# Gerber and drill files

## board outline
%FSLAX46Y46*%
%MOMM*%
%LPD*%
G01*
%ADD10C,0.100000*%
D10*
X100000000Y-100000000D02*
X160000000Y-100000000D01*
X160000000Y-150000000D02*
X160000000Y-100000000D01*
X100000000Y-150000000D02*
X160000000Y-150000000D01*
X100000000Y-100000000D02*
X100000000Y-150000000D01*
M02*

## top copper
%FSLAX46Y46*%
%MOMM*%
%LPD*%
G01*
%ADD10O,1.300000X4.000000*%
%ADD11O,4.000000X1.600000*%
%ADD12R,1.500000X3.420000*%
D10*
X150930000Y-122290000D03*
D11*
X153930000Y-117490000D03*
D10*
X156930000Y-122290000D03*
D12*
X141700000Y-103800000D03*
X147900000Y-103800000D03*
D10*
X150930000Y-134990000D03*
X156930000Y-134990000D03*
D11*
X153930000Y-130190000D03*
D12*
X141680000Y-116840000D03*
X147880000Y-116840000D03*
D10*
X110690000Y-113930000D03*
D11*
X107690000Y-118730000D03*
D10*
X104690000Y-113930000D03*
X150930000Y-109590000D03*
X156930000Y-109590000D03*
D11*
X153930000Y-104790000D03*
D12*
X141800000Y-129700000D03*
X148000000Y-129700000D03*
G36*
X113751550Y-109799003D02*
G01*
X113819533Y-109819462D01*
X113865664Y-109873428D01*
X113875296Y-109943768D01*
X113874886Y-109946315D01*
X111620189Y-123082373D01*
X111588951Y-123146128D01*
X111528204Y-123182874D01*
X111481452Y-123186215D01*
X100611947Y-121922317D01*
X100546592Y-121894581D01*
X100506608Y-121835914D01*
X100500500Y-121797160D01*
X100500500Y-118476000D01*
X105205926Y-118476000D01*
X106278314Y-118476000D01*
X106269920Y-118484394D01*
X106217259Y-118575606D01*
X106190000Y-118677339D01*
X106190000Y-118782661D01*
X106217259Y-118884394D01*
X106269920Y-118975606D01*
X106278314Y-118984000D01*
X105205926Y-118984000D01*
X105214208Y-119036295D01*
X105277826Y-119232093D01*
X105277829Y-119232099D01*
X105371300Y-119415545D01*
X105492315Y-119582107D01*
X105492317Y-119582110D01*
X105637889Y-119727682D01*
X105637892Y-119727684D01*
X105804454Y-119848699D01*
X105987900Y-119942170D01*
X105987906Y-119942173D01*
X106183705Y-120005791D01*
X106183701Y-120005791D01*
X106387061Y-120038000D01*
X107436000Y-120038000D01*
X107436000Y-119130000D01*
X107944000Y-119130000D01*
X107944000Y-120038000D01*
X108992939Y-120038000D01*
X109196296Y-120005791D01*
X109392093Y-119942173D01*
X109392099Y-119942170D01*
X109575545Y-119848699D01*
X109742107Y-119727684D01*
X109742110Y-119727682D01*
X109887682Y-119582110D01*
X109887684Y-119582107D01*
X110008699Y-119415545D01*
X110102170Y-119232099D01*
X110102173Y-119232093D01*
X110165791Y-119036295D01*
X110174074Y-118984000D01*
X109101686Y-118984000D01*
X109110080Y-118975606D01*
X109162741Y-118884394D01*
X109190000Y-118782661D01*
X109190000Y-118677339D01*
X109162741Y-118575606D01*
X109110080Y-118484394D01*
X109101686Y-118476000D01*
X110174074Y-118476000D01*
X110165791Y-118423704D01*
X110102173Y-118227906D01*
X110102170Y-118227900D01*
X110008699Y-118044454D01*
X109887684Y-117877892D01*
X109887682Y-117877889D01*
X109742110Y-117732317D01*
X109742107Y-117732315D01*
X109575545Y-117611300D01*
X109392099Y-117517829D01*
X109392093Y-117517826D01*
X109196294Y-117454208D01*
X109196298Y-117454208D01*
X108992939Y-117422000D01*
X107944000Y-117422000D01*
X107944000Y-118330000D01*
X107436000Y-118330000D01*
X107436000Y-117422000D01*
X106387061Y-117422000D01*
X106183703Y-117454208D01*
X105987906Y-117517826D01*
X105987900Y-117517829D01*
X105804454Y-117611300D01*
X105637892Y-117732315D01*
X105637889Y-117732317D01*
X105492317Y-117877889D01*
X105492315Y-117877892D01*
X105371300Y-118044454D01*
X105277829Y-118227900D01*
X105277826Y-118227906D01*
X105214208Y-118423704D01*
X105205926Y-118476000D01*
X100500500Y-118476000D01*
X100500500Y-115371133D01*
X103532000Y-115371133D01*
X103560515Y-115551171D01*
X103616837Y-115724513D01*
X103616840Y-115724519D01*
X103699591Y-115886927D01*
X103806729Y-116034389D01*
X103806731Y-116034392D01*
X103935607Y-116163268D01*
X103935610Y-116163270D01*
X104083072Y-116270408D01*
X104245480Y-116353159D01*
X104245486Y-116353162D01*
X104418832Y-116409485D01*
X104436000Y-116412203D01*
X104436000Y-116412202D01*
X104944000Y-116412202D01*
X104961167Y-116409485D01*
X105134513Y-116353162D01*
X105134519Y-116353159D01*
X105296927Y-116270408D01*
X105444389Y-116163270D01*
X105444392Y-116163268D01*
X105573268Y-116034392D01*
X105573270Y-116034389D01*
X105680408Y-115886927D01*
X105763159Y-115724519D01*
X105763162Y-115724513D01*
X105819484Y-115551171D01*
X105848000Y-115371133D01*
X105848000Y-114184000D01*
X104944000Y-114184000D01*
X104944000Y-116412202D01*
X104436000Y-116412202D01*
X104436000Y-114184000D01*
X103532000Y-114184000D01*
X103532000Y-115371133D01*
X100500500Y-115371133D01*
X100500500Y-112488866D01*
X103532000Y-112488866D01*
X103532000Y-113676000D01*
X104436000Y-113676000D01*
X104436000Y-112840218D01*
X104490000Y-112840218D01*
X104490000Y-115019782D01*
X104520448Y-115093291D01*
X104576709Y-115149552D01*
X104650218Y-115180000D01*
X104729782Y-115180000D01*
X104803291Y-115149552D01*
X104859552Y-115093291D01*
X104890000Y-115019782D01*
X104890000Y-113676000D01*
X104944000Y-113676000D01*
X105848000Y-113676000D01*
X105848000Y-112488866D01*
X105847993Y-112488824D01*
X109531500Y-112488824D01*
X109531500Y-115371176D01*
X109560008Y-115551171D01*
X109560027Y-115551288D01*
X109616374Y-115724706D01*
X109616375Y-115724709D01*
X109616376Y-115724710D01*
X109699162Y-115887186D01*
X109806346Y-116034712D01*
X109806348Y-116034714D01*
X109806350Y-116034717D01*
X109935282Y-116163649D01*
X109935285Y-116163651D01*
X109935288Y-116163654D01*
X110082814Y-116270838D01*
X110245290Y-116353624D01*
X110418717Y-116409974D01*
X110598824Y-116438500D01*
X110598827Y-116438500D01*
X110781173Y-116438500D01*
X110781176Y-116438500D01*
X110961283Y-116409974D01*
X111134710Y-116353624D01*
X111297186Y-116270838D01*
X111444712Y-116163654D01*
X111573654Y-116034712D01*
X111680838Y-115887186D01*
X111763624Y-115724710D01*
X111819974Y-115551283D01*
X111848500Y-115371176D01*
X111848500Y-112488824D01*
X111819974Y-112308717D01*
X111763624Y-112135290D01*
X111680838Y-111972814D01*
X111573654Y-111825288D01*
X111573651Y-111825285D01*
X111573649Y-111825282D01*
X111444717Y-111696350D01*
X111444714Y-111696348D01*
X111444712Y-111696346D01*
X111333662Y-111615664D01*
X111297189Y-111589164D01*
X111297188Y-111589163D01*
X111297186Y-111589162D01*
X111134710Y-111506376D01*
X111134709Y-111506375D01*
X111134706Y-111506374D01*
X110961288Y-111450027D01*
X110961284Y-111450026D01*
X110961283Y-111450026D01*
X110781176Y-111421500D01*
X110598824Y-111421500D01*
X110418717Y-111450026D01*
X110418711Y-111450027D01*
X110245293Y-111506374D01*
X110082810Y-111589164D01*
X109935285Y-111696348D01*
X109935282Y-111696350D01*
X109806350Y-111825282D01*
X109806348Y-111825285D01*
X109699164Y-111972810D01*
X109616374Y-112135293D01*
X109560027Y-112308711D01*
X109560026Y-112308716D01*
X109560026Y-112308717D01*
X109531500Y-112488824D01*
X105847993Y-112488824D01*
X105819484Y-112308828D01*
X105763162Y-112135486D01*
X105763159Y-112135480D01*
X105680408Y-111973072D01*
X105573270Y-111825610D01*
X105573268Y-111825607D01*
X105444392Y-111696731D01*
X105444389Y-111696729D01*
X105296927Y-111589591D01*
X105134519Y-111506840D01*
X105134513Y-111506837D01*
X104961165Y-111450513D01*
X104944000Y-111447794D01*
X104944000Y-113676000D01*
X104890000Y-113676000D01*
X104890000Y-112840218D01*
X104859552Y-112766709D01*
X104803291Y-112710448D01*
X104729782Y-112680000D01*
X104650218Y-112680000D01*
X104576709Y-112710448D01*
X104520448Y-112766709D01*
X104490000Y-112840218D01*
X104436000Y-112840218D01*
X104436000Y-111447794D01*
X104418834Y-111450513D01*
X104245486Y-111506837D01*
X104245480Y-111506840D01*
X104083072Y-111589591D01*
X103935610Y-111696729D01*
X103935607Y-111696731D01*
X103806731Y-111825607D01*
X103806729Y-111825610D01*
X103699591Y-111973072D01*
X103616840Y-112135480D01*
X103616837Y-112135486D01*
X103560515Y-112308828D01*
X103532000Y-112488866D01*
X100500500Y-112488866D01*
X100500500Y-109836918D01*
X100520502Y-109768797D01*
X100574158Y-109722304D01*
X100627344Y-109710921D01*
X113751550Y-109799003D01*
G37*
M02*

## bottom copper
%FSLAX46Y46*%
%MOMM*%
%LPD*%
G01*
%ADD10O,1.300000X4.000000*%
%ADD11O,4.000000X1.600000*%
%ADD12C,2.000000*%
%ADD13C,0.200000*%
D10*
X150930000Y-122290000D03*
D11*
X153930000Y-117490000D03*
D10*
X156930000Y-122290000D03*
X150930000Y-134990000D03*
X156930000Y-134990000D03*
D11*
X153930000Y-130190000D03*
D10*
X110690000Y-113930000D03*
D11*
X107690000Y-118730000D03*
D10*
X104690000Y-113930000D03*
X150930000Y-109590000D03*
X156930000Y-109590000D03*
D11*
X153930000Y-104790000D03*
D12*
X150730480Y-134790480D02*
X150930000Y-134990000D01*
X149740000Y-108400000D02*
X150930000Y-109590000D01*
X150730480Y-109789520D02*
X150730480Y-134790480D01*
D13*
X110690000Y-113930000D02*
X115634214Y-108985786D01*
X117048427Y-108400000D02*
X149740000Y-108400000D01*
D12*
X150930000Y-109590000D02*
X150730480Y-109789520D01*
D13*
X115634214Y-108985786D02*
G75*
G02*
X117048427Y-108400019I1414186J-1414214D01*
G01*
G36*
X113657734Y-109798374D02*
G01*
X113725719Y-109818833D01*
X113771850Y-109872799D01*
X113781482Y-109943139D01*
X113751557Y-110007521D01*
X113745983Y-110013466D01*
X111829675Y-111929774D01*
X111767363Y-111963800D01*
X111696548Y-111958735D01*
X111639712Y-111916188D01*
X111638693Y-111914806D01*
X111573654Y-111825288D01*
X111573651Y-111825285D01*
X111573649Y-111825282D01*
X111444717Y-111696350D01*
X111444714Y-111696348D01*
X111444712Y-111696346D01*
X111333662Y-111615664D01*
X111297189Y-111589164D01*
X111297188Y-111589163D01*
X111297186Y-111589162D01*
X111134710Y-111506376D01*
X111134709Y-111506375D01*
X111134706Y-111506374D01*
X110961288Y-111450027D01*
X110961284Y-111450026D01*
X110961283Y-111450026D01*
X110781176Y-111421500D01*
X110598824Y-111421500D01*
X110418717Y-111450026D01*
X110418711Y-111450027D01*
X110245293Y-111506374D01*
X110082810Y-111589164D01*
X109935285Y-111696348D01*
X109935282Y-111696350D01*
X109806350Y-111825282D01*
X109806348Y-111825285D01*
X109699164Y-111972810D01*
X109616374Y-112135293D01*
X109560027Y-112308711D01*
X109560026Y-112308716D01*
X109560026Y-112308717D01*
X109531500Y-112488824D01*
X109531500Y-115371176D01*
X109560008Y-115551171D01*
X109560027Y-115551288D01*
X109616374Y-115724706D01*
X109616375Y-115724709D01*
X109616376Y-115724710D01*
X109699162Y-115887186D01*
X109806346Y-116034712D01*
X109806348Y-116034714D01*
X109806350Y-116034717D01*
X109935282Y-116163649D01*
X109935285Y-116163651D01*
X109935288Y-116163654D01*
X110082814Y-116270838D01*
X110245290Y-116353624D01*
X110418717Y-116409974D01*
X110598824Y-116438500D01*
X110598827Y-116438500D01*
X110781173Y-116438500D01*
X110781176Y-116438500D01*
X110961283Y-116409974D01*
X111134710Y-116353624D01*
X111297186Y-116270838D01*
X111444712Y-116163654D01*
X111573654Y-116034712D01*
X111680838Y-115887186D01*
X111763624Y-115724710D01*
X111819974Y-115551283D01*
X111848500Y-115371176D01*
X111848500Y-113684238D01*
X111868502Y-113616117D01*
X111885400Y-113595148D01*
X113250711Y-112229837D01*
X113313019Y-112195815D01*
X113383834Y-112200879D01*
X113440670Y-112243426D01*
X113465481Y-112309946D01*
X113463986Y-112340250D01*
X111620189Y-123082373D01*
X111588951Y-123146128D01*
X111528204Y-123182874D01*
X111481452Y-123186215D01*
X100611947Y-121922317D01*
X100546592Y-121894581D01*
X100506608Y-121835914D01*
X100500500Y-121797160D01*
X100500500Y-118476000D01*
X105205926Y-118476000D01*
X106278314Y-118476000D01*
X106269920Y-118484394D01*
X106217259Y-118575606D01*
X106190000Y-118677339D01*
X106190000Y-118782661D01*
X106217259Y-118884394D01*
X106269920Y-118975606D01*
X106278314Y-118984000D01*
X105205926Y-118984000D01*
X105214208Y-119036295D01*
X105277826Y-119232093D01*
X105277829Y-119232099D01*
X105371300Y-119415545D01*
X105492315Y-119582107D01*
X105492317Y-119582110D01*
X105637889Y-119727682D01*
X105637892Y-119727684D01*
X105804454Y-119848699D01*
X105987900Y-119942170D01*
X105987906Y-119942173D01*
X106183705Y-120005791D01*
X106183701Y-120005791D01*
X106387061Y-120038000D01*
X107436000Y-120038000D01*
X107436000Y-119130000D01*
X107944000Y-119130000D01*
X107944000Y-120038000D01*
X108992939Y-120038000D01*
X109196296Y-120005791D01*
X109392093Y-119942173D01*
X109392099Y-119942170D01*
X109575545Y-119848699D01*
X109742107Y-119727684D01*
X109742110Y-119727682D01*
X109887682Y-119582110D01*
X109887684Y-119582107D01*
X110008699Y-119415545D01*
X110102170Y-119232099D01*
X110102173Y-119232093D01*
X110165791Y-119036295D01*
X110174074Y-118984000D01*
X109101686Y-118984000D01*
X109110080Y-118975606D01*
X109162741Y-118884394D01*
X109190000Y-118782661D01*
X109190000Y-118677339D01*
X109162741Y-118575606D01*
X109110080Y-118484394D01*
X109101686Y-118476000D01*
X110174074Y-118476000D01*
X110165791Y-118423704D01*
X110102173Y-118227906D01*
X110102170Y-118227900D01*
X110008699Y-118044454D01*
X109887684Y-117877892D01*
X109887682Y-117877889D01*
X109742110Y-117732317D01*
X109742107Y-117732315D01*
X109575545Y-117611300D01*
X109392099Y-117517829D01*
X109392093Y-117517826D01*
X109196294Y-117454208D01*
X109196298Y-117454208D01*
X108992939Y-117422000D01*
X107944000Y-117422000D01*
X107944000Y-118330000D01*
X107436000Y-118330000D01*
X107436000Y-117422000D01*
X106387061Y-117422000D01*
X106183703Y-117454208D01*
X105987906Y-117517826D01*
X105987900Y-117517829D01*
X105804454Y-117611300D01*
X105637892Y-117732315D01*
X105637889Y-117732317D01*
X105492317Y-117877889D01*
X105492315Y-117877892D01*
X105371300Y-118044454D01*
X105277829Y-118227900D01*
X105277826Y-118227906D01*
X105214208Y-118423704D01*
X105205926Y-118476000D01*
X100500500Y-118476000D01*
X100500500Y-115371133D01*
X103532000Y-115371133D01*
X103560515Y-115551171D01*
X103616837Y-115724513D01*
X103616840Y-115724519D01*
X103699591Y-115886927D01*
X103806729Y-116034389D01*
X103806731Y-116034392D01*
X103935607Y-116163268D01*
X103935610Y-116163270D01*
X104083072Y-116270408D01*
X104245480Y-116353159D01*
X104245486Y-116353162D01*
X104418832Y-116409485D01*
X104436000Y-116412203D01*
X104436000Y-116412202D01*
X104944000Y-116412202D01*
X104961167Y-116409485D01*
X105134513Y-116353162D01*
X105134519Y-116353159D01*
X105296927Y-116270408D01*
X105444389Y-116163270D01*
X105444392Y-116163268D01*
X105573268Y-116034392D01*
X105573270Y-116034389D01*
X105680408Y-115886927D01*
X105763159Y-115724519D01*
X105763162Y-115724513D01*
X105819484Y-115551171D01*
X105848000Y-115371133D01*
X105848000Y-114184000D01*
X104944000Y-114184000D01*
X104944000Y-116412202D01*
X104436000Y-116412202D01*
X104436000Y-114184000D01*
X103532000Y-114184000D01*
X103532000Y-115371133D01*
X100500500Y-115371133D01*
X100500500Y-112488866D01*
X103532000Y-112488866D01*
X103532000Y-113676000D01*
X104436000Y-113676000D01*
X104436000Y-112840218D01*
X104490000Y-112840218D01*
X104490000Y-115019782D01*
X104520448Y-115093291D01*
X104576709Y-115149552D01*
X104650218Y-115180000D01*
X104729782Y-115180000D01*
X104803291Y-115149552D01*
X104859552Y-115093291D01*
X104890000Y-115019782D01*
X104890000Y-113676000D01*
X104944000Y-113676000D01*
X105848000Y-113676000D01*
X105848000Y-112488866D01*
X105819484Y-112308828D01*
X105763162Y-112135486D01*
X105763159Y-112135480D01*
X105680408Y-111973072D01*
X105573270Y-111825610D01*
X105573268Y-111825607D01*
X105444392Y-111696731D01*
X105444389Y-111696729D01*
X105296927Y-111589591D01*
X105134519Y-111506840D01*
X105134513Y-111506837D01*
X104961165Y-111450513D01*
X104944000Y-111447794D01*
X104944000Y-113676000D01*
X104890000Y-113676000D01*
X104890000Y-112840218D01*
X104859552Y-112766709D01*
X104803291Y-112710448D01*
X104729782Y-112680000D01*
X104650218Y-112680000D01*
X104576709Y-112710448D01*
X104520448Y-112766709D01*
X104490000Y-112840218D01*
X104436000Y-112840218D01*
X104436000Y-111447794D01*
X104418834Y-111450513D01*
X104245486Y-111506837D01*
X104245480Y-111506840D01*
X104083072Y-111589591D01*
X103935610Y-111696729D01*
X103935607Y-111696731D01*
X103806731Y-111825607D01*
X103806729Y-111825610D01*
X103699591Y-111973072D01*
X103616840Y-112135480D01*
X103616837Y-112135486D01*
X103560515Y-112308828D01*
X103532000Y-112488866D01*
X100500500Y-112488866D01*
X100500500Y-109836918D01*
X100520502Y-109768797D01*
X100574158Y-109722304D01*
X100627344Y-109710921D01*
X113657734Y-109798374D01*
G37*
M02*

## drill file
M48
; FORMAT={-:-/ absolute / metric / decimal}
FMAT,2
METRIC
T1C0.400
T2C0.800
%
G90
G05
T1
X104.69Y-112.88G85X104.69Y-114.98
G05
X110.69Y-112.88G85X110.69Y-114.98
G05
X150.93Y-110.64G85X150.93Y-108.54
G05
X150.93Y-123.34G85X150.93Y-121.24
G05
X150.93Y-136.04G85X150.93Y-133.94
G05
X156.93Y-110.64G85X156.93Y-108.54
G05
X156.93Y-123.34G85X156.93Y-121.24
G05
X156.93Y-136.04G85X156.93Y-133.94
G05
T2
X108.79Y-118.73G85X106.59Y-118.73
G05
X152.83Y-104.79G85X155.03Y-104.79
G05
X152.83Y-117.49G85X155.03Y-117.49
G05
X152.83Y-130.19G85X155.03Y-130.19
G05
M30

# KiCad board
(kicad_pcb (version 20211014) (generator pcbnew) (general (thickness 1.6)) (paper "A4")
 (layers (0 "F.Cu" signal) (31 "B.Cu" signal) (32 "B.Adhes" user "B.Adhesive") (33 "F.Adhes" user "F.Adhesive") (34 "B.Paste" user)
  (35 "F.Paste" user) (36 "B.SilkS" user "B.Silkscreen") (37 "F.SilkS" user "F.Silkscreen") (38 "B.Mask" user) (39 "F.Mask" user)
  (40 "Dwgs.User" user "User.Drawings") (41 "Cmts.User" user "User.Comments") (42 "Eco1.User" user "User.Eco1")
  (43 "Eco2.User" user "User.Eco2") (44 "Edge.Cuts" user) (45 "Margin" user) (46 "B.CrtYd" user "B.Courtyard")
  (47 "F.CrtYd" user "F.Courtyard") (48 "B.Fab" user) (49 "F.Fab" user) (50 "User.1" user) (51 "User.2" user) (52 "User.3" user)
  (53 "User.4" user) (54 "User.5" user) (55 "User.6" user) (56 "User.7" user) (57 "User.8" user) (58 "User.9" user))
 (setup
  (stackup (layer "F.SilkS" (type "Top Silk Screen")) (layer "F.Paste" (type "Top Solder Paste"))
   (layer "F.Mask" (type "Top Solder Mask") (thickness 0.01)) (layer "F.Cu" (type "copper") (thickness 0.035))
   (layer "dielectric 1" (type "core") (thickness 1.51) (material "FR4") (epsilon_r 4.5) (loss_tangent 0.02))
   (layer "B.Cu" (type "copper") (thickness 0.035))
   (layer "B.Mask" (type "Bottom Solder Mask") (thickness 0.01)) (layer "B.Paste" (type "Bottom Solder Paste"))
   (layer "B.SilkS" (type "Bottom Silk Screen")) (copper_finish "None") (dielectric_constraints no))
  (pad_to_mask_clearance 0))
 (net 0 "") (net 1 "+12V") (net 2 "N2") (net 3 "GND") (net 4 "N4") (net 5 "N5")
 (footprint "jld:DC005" (layer "F.Cu") (at 164.43 122.29 90)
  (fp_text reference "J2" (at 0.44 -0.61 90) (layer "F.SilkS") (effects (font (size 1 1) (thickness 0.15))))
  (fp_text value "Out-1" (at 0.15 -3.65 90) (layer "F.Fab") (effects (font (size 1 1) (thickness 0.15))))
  (pad "1" thru_hole oval locked (at 0 -13.5 90) (size 4 1.3) (drill oval 2.5 0.4) (layers *.Cu *.Mask) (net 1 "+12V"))
  (pad "2" thru_hole oval locked (at 4.8 -10.5 90) (size 1.6 4) (drill oval 0.8 3) (layers *.Cu *.Mask) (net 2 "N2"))
  (pad "2" thru_hole oval locked (at 0 -7.5 90) (size 4 1.3) (drill oval 2.5 0.4) (layers *.Cu *.Mask) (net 2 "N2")))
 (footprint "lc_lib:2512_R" (layer "F.Cu") (at 144.8 103.8)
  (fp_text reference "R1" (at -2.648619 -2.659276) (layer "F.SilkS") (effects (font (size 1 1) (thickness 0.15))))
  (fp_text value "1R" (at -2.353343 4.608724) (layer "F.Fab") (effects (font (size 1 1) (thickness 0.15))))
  (pad "1" smd rect locked (at -3.1 0) (size 1.5 3.42) (layers "F.Cu" "F.Paste" "F.Mask") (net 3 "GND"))
  (pad "2" smd rect locked (at 3.1 0) (size 1.5 3.42) (layers "F.Cu" "F.Paste" "F.Mask") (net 2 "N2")))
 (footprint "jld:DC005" (layer "F.Cu") (at 164.43 134.99 90)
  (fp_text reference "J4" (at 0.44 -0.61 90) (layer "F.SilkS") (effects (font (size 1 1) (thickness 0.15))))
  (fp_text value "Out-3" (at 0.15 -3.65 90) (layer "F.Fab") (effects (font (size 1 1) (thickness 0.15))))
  (pad "1" thru_hole oval locked (at 0 -13.5 90) (size 4 1.3) (drill oval 2.5 0.4) (layers *.Cu *.Mask) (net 1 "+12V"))
  (pad "2" thru_hole oval locked (at 0 -7.5 90) (size 4 1.3) (drill oval 2.5 0.4) (layers *.Cu *.Mask) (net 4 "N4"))
  (pad "2" thru_hole oval locked (at 4.8 -10.5 90) (size 1.6 4) (drill oval 0.8 3) (layers *.Cu *.Mask) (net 4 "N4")))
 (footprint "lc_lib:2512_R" (layer "F.Cu") (at 144.78 116.84)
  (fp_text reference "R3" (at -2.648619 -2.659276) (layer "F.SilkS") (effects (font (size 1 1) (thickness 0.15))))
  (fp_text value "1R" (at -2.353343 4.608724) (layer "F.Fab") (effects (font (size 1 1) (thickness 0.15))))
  (pad "1" smd rect locked (at -3.1 0) (size 1.5 3.42) (layers "F.Cu" "F.Paste" "F.Mask") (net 3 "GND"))
  (pad "2" smd rect locked (at 3.1 0) (size 1.5 3.42) (layers "F.Cu" "F.Paste" "F.Mask") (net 4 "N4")))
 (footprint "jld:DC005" (layer "F.Cu") (at 97.19 113.93 -90)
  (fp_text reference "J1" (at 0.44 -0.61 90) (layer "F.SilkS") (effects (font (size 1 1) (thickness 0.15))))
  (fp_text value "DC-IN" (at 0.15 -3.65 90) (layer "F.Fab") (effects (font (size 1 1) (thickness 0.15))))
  (pad "1" thru_hole oval locked (at 0 -13.5 270) (size 4 1.3) (drill oval 2.5 0.4) (layers *.Cu *.Mask) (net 1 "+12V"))
  (pad "2" thru_hole oval locked (at 4.8 -10.5 270) (size 1.6 4) (drill oval 0.8 3) (layers *.Cu *.Mask) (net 3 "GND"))
  (pad "2" thru_hole oval locked (at 0 -7.5 270) (size 4 1.3) (drill oval 2.5 0.4) (layers *.Cu *.Mask) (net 3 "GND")))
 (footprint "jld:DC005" (layer "F.Cu") (at 164.43 109.59 90)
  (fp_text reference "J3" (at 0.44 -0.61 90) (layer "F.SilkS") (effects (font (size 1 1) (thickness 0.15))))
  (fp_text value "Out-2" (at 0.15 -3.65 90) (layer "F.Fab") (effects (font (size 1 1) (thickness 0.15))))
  (pad "1" thru_hole oval locked (at 0 -13.5 90) (size 4 1.3) (drill oval 2.5 0.4) (layers *.Cu *.Mask) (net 1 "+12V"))
  (pad "2" thru_hole oval locked (at 0 -7.5 90) (size 4 1.3) (drill oval 2.5 0.4) (layers *.Cu *.Mask) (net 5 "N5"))
  (pad "2" thru_hole oval locked (at 4.8 -10.5 90) (size 1.6 4) (drill oval 0.8 3) (layers *.Cu *.Mask) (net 5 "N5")))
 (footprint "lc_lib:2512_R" (layer "F.Cu") (at 144.9 129.7)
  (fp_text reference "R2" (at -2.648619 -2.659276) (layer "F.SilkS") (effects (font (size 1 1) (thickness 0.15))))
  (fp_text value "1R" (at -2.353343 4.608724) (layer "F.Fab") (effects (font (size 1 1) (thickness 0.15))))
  (pad "1" smd rect locked (at -3.1 0) (size 1.5 3.42) (layers "F.Cu" "F.Paste" "F.Mask") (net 3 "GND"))
  (pad "2" smd rect locked (at 3.1 0) (size 1.5 3.42) (layers "F.Cu" "F.Paste" "F.Mask") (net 5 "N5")))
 (gr_line (start 100 100) (end 160 100) (layer "Edge.Cuts") (width 0.1))
 (gr_line (start 160 150) (end 160 100) (layer "Edge.Cuts") (width 0.1))
 (gr_line (start 100 150) (end 160 150) (layer "Edge.Cuts") (width 0.1))
 (gr_line (start 100 100) (end 100 150) (layer "Edge.Cuts") (width 0.1))
 (segment (start 150.73048 134.79048) (end 150.93 134.99) (width 2) (layer "B.Cu") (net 1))
 (segment (start 149.74 108.4) (end 150.93 109.59) (width 2) (layer "B.Cu") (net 1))
 (segment (start 150.73048 109.78952) (end 150.73048 134.79048) (width 2) (layer "B.Cu") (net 1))
 (segment (start 110.69 113.93) (end 115.634214 108.985786) (width 0.2) (layer "B.Cu") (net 1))
 (segment (start 117.048427 108.4) (end 149.74 108.4) (width 0.2) (layer "B.Cu") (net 1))
 (segment (start 150.93 109.59) (end 150.73048 109.78952) (width 2) (layer "B.Cu") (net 1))
 (arc (start 115.634214 108.985786) (mid 116.28306 108.552241) (end 117.048427 108.4) (width 0.2) (layer "B.Cu") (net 1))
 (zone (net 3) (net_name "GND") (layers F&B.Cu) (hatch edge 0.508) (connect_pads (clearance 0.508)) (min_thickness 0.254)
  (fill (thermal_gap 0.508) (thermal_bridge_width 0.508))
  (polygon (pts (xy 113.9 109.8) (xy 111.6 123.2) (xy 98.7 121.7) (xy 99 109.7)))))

